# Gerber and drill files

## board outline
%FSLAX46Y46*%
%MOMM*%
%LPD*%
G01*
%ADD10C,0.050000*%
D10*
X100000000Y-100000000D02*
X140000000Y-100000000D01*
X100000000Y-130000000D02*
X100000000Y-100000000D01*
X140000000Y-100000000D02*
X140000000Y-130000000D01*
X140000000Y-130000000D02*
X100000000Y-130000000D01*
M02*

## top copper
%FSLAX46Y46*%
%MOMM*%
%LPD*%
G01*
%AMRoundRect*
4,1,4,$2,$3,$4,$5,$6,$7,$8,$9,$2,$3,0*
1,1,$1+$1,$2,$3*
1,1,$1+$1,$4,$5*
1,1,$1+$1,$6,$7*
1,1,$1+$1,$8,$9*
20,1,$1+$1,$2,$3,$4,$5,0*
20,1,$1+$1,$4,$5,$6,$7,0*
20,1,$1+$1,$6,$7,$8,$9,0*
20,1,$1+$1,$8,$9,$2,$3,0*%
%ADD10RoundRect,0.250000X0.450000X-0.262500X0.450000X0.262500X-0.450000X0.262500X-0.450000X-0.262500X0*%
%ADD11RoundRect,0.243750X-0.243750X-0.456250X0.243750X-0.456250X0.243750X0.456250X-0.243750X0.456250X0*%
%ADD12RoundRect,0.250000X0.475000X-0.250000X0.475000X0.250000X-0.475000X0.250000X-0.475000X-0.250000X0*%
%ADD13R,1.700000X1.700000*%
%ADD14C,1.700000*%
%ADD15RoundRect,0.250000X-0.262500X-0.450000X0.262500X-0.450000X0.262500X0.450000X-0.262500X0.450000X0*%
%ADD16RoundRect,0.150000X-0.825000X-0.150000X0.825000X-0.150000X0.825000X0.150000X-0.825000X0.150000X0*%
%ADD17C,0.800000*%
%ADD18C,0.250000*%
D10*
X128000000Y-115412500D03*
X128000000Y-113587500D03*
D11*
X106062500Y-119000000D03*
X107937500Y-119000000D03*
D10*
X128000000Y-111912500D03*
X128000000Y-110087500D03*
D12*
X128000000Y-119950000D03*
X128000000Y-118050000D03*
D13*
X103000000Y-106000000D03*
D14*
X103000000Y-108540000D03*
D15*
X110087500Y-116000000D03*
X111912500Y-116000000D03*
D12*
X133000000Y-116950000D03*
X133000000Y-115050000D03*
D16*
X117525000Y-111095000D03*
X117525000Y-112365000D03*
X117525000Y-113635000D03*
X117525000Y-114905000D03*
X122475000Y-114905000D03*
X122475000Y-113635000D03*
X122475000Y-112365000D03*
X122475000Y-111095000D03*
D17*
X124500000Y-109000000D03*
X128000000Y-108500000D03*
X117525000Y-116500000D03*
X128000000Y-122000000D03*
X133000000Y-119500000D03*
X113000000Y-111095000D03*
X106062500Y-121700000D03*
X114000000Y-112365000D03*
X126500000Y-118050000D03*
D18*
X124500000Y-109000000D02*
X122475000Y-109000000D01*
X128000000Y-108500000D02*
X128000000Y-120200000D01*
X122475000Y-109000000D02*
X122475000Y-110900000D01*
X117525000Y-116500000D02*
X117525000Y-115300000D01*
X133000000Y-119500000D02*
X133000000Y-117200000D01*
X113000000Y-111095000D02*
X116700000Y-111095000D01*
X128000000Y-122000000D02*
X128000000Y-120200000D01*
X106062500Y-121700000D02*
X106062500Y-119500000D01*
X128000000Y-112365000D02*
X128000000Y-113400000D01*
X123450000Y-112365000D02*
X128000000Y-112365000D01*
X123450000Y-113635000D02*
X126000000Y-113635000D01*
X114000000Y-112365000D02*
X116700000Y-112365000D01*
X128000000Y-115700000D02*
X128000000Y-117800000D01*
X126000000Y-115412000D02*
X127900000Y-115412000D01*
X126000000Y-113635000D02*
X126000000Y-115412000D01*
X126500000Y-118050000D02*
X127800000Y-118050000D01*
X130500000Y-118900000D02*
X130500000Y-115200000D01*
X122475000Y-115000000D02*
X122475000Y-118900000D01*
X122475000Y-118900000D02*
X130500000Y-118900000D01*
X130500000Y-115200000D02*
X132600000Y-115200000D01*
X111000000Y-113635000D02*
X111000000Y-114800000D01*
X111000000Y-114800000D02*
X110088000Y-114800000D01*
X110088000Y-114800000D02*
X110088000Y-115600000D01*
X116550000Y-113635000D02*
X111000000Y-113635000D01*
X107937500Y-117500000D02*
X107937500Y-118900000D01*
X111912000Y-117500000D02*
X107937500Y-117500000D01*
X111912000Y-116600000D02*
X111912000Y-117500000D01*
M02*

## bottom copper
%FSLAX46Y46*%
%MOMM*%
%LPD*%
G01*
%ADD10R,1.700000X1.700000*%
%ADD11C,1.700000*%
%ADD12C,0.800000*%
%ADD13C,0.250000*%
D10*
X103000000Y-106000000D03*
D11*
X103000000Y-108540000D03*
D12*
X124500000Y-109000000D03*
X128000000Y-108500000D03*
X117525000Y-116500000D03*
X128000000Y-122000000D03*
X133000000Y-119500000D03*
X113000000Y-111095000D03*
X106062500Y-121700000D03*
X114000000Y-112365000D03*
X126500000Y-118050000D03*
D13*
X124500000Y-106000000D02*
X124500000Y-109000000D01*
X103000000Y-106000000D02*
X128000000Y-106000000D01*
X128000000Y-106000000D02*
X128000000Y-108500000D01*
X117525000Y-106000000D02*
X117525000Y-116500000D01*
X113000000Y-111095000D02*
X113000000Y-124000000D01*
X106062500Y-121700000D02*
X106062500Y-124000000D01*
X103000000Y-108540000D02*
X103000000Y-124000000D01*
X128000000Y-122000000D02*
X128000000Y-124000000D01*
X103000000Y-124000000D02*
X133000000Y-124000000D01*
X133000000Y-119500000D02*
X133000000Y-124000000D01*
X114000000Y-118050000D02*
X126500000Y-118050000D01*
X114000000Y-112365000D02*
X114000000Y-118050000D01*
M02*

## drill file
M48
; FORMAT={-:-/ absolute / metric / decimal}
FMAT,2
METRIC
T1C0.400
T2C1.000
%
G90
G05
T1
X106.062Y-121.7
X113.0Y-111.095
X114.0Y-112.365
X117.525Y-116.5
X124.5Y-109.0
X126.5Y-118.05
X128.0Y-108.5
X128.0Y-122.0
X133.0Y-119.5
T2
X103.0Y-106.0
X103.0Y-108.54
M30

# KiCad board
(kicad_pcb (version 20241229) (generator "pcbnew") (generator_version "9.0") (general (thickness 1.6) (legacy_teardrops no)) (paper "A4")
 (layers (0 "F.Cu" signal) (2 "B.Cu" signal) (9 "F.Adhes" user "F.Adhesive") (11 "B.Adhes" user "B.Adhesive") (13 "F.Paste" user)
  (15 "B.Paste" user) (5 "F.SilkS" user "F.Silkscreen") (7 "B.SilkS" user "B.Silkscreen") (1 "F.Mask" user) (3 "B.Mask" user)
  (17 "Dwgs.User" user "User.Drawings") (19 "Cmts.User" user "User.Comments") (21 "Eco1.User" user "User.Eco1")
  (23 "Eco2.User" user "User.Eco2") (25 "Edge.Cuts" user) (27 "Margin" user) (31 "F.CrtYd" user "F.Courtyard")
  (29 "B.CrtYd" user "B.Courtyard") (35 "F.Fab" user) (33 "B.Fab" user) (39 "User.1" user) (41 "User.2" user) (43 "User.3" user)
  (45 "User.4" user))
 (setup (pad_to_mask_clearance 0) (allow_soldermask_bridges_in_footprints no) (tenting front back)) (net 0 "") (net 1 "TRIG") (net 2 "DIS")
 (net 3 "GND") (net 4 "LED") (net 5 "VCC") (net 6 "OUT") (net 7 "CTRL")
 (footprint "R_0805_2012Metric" (layer "F.Cu") (at 128 114.5 90)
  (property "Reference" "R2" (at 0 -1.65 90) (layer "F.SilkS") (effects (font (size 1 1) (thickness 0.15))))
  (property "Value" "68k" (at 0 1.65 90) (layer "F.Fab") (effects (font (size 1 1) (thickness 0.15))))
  (pad "1" smd roundrect (at -0.9125 0 90) (size 1.025 1.4) (layers "F.Cu" "F.Mask" "F.Paste") (roundrect_rratio 0.243902) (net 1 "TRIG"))
  (pad "2" smd roundrect (at 0.9125 0 90) (size 1.025 1.4) (layers "F.Cu" "F.Mask" "F.Paste") (roundrect_rratio 0.243902) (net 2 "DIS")))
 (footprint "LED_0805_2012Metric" (layer "F.Cu") (at 107 119)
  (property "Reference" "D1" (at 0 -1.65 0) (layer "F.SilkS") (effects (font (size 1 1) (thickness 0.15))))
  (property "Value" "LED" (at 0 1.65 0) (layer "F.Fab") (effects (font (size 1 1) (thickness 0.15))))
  (pad "1" smd roundrect (at -0.9375 0) (size 0.975 1.4) (layers "F.Cu" "F.Mask" "F.Paste") (roundrect_rratio 0.25) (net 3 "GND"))
  (pad "2" smd roundrect (at 0.9375 0) (size 0.975 1.4) (layers "F.Cu" "F.Mask" "F.Paste") (roundrect_rratio 0.25) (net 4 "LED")))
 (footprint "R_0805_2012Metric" (layer "F.Cu") (at 128 111 90)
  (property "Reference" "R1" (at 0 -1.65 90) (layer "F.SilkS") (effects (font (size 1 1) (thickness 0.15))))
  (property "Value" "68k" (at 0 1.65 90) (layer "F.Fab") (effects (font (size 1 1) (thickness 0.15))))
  (pad "1" smd roundrect (at -0.9125 0 90) (size 1.025 1.4) (layers "F.Cu" "F.Mask" "F.Paste") (roundrect_rratio 0.243902) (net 2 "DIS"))
  (pad "2" smd roundrect (at 0.9125 0 90) (size 1.025 1.4) (layers "F.Cu" "F.Mask" "F.Paste") (roundrect_rratio 0.243902) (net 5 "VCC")))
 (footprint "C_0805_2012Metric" (layer "F.Cu") (at 128 119 90)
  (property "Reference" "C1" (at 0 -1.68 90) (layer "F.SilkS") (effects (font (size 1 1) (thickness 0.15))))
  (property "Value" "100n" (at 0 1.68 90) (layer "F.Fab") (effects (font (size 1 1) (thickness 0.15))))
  (pad "1" smd roundrect (at -0.95 0 90) (size 1 1.45) (layers "F.Cu" "F.Mask" "F.Paste") (roundrect_rratio 0.25) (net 3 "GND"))
  (pad "2" smd roundrect (at 0.95 0 90) (size 1 1.45) (layers "F.Cu" "F.Mask" "F.Paste") (roundrect_rratio 0.25) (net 1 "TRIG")))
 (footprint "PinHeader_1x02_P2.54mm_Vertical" (layer "F.Cu") (at 103 106)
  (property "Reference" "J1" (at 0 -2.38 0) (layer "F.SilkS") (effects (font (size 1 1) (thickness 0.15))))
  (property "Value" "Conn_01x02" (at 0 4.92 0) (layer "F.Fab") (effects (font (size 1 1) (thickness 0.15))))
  (pad "1" thru_hole rect (at 0 0) (size 1.7 1.7) (drill 1) (layers "*.Cu" "*.Mask") (remove_unused_layers no) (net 5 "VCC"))
  (pad "2" thru_hole circle (at 0 2.54) (size 1.7 1.7) (drill 1) (layers "*.Cu" "*.Mask") (remove_unused_layers no) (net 3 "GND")))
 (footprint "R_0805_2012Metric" (layer "F.Cu") (at 111 116)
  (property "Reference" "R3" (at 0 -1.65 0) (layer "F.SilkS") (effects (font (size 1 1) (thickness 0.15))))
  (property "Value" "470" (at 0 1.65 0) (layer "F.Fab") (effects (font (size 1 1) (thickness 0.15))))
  (pad "1" smd roundrect (at -0.9125 0) (size 1.025 1.4) (layers "F.Cu" "F.Mask" "F.Paste") (roundrect_rratio 0.243902) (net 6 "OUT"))
  (pad "2" smd roundrect (at 0.9125 0) (size 1.025 1.4) (layers "F.Cu" "F.Mask" "F.Paste") (roundrect_rratio 0.243902) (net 4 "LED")))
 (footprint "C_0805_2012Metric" (layer "F.Cu") (at 133 116 90)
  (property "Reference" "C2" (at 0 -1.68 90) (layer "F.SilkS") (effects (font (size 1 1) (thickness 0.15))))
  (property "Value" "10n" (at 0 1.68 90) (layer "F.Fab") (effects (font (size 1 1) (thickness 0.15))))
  (pad "1" smd roundrect (at -0.95 0 90) (size 1 1.45) (layers "F.Cu" "F.Mask" "F.Paste") (roundrect_rratio 0.25) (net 3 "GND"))
  (pad "2" smd roundrect (at 0.95 0 90) (size 1 1.45) (layers "F.Cu" "F.Mask" "F.Paste") (roundrect_rratio 0.25) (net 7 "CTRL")))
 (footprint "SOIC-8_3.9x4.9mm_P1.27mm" (layer "F.Cu") (at 120 113)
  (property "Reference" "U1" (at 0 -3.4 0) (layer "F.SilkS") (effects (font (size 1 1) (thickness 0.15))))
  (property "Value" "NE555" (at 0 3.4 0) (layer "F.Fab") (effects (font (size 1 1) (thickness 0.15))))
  (pad "1" smd roundrect (at -2.475 -1.905) (size 1.95 0.6) (layers "F.Cu" "F.Mask" "F.Paste") (roundrect_rratio 0.25) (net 3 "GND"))
  (pad "2" smd roundrect (at -2.475 -0.635) (size 1.95 0.6) (layers "F.Cu" "F.Mask" "F.Paste") (roundrect_rratio 0.25) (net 1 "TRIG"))
  (pad "3" smd roundrect (at -2.475 0.635) (size 1.95 0.6) (layers "F.Cu" "F.Mask" "F.Paste") (roundrect_rratio 0.25) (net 6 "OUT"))
  (pad "4" smd roundrect (at -2.475 1.905) (size 1.95 0.6) (layers "F.Cu" "F.Mask" "F.Paste") (roundrect_rratio 0.25) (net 5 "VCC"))
  (pad "5" smd roundrect (at 2.475 1.905) (size 1.95 0.6) (layers "F.Cu" "F.Mask" "F.Paste") (roundrect_rratio 0.25) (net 7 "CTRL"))
  (pad "6" smd roundrect (at 2.475 0.635) (size 1.95 0.6) (layers "F.Cu" "F.Mask" "F.Paste") (roundrect_rratio 0.25) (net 1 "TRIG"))
  (pad "7" smd roundrect (at 2.475 -0.635) (size 1.95 0.6) (layers "F.Cu" "F.Mask" "F.Paste") (roundrect_rratio 0.25) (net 2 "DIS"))
  (pad "8" smd roundrect (at 2.475 -1.905) (size 1.95 0.6) (layers "F.Cu" "F.Mask" "F.Paste") (roundrect_rratio 0.25) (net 5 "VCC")))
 (gr_line (start 100 100) (end 140 100) (stroke (width 0.05) (type default)) (layer "Edge.Cuts"))
 (gr_line (start 100 130) (end 100 100) (stroke (width 0.05) (type default)) (layer "Edge.Cuts"))
 (gr_line (start 140 100) (end 140 130) (stroke (width 0.05) (type default)) (layer "Edge.Cuts"))
 (gr_line (start 140 130) (end 100 130) (stroke (width 0.05) (type default)) (layer "Edge.Cuts"))
 (segment (start 124.5 109) (end 122.475 109) (width 0.25) (layer "F.Cu") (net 5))
 (segment (start 128 108.5) (end 128 120.2) (width 0.25) (layer "F.Cu") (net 5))
 (segment (start 122.475 109) (end 122.475 110.9) (width 0.25) (layer "F.Cu") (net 5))
 (segment (start 117.525 116.5) (end 117.525 115.3) (width 0.25) (layer "F.Cu") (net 5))
 (via (at 124.5 109) (size 0.8) (drill 0.4) (layers "F.Cu" "B.Cu") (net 5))
 (via (at 128 108.5) (size 0.8) (drill 0.4) (layers "F.Cu" "B.Cu") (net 5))
 (via (at 117.525 116.5) (size 0.8) (drill 0.4) (layers "F.Cu" "B.Cu") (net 5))
 (segment (start 124.5 106) (end 124.5 109) (width 0.25) (layer "B.Cu") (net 5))
 (segment (start 103 106) (end 128 106) (width 0.25) (layer "B.Cu") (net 5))
 (segment (start 128 106) (end 128 108.5) (width 0.25) (layer "B.Cu") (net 5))
 (segment (start 117.525 106) (end 117.525 116.5) (width 0.25) (layer "B.Cu") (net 5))
 (segment (start 133 119.5) (end 133 117.2) (width 0.25) (layer "F.Cu") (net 3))
 (segment (start 113 111.095) (end 116.7 111.095) (width 0.25) (layer "F.Cu") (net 3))
 (segment (start 128 122) (end 128 120.2) (width 0.25) (layer "F.Cu") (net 3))
 (segment (start 106.0625 121.7) (end 106.0625 119.5) (width 0.25) (layer "F.Cu") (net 3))
 (via (at 128 122) (size 0.8) (drill 0.4) (layers "F.Cu" "B.Cu") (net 3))
 (via (at 133 119.5) (size 0.8) (drill 0.4) (layers "F.Cu" "B.Cu") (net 3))
 (via (at 113 111.095) (size 0.8) (drill 0.4) (layers "F.Cu" "B.Cu") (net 3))
 (via (at 106.0625 121.7) (size 0.8) (drill 0.4) (layers "F.Cu" "B.Cu") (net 3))
 (segment (start 113 111.095) (end 113 124) (width 0.25) (layer "B.Cu") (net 3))
 (segment (start 106.0625 121.7) (end 106.0625 124) (width 0.25) (layer "B.Cu") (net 3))
 (segment (start 103 108.54) (end 103 124) (width 0.25) (layer "B.Cu") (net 3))
 (segment (start 128 122) (end 128 124) (width 0.25) (layer "B.Cu") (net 3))
 (segment (start 103 124) (end 133 124) (width 0.25) (layer "B.Cu") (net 3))
 (segment (start 133 119.5) (end 133 124) (width 0.25) (layer "B.Cu") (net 3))
 (segment (start 128 112.365) (end 128 113.4) (width 0.25) (layer "F.Cu") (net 2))
 (segment (start 123.45 112.365) (end 128 112.365) (width 0.25) (layer "F.Cu") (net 2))
 (segment (start 123.45 113.635) (end 126 113.635) (width 0.25) (layer "F.Cu") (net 1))
 (segment (start 114 112.365) (end 116.7 112.365) (width 0.25) (layer "F.Cu") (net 1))
 (segment (start 128 115.7) (end 128 117.8) (width 0.25) (layer "F.Cu") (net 1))
 (segment (start 126 115.412) (end 127.9 115.412) (width 0.25) (layer "F.Cu") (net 1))
 (segment (start 126 113.635) (end 126 115.412) (width 0.25) (layer "F.Cu") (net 1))
 (segment (start 126.5 118.05) (end 127.8 118.05) (width 0.25) (layer "F.Cu") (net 1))
 (via (at 114 112.365) (size 0.8) (drill 0.4) (layers "F.Cu" "B.Cu") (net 1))
 (via (at 126.5 118.05) (size 0.8) (drill 0.4) (layers "F.Cu" "B.Cu") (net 1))
 (segment (start 114 118.05) (end 126.5 118.05) (width 0.25) (layer "B.Cu") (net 1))
 (segment (start 114 112.365) (end 114 118.05) (width 0.25) (layer "B.Cu") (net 1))
 (segment (start 130.5 118.9) (end 130.5 115.2) (width 0.25) (layer "F.Cu") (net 7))
 (segment (start 122.475 115) (end 122.475 118.9) (width 0.25) (layer "F.Cu") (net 7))
 (segment (start 122.475 118.9) (end 130.5 118.9) (width 0.25) (layer "F.Cu") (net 7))
 (segment (start 130.5 115.2) (end 132.6 115.2) (width 0.25) (layer "F.Cu") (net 7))
 (segment (start 111 113.635) (end 111 114.8) (width 0.25) (layer "F.Cu") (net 6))
 (segment (start 111 114.8) (end 110.088 114.8) (width 0.25) (layer "F.Cu") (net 6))
 (segment (start 110.088 114.8) (end 110.088 115.6) (width 0.25) (layer "F.Cu") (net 6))
 (segment (start 116.55 113.635) (end 111 113.635) (width 0.25) (layer "F.Cu") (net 6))
 (segment (start 107.9375 117.5) (end 107.9375 118.9) (width 0.25) (layer "F.Cu") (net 4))
 (segment (start 111.912 117.5) (end 107.9375 117.5) (width 0.25) (layer "F.Cu") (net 4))
 (segment (start 111.912 116.6) (end 111.912 117.5) (width 0.25) (layer "F.Cu") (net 4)))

